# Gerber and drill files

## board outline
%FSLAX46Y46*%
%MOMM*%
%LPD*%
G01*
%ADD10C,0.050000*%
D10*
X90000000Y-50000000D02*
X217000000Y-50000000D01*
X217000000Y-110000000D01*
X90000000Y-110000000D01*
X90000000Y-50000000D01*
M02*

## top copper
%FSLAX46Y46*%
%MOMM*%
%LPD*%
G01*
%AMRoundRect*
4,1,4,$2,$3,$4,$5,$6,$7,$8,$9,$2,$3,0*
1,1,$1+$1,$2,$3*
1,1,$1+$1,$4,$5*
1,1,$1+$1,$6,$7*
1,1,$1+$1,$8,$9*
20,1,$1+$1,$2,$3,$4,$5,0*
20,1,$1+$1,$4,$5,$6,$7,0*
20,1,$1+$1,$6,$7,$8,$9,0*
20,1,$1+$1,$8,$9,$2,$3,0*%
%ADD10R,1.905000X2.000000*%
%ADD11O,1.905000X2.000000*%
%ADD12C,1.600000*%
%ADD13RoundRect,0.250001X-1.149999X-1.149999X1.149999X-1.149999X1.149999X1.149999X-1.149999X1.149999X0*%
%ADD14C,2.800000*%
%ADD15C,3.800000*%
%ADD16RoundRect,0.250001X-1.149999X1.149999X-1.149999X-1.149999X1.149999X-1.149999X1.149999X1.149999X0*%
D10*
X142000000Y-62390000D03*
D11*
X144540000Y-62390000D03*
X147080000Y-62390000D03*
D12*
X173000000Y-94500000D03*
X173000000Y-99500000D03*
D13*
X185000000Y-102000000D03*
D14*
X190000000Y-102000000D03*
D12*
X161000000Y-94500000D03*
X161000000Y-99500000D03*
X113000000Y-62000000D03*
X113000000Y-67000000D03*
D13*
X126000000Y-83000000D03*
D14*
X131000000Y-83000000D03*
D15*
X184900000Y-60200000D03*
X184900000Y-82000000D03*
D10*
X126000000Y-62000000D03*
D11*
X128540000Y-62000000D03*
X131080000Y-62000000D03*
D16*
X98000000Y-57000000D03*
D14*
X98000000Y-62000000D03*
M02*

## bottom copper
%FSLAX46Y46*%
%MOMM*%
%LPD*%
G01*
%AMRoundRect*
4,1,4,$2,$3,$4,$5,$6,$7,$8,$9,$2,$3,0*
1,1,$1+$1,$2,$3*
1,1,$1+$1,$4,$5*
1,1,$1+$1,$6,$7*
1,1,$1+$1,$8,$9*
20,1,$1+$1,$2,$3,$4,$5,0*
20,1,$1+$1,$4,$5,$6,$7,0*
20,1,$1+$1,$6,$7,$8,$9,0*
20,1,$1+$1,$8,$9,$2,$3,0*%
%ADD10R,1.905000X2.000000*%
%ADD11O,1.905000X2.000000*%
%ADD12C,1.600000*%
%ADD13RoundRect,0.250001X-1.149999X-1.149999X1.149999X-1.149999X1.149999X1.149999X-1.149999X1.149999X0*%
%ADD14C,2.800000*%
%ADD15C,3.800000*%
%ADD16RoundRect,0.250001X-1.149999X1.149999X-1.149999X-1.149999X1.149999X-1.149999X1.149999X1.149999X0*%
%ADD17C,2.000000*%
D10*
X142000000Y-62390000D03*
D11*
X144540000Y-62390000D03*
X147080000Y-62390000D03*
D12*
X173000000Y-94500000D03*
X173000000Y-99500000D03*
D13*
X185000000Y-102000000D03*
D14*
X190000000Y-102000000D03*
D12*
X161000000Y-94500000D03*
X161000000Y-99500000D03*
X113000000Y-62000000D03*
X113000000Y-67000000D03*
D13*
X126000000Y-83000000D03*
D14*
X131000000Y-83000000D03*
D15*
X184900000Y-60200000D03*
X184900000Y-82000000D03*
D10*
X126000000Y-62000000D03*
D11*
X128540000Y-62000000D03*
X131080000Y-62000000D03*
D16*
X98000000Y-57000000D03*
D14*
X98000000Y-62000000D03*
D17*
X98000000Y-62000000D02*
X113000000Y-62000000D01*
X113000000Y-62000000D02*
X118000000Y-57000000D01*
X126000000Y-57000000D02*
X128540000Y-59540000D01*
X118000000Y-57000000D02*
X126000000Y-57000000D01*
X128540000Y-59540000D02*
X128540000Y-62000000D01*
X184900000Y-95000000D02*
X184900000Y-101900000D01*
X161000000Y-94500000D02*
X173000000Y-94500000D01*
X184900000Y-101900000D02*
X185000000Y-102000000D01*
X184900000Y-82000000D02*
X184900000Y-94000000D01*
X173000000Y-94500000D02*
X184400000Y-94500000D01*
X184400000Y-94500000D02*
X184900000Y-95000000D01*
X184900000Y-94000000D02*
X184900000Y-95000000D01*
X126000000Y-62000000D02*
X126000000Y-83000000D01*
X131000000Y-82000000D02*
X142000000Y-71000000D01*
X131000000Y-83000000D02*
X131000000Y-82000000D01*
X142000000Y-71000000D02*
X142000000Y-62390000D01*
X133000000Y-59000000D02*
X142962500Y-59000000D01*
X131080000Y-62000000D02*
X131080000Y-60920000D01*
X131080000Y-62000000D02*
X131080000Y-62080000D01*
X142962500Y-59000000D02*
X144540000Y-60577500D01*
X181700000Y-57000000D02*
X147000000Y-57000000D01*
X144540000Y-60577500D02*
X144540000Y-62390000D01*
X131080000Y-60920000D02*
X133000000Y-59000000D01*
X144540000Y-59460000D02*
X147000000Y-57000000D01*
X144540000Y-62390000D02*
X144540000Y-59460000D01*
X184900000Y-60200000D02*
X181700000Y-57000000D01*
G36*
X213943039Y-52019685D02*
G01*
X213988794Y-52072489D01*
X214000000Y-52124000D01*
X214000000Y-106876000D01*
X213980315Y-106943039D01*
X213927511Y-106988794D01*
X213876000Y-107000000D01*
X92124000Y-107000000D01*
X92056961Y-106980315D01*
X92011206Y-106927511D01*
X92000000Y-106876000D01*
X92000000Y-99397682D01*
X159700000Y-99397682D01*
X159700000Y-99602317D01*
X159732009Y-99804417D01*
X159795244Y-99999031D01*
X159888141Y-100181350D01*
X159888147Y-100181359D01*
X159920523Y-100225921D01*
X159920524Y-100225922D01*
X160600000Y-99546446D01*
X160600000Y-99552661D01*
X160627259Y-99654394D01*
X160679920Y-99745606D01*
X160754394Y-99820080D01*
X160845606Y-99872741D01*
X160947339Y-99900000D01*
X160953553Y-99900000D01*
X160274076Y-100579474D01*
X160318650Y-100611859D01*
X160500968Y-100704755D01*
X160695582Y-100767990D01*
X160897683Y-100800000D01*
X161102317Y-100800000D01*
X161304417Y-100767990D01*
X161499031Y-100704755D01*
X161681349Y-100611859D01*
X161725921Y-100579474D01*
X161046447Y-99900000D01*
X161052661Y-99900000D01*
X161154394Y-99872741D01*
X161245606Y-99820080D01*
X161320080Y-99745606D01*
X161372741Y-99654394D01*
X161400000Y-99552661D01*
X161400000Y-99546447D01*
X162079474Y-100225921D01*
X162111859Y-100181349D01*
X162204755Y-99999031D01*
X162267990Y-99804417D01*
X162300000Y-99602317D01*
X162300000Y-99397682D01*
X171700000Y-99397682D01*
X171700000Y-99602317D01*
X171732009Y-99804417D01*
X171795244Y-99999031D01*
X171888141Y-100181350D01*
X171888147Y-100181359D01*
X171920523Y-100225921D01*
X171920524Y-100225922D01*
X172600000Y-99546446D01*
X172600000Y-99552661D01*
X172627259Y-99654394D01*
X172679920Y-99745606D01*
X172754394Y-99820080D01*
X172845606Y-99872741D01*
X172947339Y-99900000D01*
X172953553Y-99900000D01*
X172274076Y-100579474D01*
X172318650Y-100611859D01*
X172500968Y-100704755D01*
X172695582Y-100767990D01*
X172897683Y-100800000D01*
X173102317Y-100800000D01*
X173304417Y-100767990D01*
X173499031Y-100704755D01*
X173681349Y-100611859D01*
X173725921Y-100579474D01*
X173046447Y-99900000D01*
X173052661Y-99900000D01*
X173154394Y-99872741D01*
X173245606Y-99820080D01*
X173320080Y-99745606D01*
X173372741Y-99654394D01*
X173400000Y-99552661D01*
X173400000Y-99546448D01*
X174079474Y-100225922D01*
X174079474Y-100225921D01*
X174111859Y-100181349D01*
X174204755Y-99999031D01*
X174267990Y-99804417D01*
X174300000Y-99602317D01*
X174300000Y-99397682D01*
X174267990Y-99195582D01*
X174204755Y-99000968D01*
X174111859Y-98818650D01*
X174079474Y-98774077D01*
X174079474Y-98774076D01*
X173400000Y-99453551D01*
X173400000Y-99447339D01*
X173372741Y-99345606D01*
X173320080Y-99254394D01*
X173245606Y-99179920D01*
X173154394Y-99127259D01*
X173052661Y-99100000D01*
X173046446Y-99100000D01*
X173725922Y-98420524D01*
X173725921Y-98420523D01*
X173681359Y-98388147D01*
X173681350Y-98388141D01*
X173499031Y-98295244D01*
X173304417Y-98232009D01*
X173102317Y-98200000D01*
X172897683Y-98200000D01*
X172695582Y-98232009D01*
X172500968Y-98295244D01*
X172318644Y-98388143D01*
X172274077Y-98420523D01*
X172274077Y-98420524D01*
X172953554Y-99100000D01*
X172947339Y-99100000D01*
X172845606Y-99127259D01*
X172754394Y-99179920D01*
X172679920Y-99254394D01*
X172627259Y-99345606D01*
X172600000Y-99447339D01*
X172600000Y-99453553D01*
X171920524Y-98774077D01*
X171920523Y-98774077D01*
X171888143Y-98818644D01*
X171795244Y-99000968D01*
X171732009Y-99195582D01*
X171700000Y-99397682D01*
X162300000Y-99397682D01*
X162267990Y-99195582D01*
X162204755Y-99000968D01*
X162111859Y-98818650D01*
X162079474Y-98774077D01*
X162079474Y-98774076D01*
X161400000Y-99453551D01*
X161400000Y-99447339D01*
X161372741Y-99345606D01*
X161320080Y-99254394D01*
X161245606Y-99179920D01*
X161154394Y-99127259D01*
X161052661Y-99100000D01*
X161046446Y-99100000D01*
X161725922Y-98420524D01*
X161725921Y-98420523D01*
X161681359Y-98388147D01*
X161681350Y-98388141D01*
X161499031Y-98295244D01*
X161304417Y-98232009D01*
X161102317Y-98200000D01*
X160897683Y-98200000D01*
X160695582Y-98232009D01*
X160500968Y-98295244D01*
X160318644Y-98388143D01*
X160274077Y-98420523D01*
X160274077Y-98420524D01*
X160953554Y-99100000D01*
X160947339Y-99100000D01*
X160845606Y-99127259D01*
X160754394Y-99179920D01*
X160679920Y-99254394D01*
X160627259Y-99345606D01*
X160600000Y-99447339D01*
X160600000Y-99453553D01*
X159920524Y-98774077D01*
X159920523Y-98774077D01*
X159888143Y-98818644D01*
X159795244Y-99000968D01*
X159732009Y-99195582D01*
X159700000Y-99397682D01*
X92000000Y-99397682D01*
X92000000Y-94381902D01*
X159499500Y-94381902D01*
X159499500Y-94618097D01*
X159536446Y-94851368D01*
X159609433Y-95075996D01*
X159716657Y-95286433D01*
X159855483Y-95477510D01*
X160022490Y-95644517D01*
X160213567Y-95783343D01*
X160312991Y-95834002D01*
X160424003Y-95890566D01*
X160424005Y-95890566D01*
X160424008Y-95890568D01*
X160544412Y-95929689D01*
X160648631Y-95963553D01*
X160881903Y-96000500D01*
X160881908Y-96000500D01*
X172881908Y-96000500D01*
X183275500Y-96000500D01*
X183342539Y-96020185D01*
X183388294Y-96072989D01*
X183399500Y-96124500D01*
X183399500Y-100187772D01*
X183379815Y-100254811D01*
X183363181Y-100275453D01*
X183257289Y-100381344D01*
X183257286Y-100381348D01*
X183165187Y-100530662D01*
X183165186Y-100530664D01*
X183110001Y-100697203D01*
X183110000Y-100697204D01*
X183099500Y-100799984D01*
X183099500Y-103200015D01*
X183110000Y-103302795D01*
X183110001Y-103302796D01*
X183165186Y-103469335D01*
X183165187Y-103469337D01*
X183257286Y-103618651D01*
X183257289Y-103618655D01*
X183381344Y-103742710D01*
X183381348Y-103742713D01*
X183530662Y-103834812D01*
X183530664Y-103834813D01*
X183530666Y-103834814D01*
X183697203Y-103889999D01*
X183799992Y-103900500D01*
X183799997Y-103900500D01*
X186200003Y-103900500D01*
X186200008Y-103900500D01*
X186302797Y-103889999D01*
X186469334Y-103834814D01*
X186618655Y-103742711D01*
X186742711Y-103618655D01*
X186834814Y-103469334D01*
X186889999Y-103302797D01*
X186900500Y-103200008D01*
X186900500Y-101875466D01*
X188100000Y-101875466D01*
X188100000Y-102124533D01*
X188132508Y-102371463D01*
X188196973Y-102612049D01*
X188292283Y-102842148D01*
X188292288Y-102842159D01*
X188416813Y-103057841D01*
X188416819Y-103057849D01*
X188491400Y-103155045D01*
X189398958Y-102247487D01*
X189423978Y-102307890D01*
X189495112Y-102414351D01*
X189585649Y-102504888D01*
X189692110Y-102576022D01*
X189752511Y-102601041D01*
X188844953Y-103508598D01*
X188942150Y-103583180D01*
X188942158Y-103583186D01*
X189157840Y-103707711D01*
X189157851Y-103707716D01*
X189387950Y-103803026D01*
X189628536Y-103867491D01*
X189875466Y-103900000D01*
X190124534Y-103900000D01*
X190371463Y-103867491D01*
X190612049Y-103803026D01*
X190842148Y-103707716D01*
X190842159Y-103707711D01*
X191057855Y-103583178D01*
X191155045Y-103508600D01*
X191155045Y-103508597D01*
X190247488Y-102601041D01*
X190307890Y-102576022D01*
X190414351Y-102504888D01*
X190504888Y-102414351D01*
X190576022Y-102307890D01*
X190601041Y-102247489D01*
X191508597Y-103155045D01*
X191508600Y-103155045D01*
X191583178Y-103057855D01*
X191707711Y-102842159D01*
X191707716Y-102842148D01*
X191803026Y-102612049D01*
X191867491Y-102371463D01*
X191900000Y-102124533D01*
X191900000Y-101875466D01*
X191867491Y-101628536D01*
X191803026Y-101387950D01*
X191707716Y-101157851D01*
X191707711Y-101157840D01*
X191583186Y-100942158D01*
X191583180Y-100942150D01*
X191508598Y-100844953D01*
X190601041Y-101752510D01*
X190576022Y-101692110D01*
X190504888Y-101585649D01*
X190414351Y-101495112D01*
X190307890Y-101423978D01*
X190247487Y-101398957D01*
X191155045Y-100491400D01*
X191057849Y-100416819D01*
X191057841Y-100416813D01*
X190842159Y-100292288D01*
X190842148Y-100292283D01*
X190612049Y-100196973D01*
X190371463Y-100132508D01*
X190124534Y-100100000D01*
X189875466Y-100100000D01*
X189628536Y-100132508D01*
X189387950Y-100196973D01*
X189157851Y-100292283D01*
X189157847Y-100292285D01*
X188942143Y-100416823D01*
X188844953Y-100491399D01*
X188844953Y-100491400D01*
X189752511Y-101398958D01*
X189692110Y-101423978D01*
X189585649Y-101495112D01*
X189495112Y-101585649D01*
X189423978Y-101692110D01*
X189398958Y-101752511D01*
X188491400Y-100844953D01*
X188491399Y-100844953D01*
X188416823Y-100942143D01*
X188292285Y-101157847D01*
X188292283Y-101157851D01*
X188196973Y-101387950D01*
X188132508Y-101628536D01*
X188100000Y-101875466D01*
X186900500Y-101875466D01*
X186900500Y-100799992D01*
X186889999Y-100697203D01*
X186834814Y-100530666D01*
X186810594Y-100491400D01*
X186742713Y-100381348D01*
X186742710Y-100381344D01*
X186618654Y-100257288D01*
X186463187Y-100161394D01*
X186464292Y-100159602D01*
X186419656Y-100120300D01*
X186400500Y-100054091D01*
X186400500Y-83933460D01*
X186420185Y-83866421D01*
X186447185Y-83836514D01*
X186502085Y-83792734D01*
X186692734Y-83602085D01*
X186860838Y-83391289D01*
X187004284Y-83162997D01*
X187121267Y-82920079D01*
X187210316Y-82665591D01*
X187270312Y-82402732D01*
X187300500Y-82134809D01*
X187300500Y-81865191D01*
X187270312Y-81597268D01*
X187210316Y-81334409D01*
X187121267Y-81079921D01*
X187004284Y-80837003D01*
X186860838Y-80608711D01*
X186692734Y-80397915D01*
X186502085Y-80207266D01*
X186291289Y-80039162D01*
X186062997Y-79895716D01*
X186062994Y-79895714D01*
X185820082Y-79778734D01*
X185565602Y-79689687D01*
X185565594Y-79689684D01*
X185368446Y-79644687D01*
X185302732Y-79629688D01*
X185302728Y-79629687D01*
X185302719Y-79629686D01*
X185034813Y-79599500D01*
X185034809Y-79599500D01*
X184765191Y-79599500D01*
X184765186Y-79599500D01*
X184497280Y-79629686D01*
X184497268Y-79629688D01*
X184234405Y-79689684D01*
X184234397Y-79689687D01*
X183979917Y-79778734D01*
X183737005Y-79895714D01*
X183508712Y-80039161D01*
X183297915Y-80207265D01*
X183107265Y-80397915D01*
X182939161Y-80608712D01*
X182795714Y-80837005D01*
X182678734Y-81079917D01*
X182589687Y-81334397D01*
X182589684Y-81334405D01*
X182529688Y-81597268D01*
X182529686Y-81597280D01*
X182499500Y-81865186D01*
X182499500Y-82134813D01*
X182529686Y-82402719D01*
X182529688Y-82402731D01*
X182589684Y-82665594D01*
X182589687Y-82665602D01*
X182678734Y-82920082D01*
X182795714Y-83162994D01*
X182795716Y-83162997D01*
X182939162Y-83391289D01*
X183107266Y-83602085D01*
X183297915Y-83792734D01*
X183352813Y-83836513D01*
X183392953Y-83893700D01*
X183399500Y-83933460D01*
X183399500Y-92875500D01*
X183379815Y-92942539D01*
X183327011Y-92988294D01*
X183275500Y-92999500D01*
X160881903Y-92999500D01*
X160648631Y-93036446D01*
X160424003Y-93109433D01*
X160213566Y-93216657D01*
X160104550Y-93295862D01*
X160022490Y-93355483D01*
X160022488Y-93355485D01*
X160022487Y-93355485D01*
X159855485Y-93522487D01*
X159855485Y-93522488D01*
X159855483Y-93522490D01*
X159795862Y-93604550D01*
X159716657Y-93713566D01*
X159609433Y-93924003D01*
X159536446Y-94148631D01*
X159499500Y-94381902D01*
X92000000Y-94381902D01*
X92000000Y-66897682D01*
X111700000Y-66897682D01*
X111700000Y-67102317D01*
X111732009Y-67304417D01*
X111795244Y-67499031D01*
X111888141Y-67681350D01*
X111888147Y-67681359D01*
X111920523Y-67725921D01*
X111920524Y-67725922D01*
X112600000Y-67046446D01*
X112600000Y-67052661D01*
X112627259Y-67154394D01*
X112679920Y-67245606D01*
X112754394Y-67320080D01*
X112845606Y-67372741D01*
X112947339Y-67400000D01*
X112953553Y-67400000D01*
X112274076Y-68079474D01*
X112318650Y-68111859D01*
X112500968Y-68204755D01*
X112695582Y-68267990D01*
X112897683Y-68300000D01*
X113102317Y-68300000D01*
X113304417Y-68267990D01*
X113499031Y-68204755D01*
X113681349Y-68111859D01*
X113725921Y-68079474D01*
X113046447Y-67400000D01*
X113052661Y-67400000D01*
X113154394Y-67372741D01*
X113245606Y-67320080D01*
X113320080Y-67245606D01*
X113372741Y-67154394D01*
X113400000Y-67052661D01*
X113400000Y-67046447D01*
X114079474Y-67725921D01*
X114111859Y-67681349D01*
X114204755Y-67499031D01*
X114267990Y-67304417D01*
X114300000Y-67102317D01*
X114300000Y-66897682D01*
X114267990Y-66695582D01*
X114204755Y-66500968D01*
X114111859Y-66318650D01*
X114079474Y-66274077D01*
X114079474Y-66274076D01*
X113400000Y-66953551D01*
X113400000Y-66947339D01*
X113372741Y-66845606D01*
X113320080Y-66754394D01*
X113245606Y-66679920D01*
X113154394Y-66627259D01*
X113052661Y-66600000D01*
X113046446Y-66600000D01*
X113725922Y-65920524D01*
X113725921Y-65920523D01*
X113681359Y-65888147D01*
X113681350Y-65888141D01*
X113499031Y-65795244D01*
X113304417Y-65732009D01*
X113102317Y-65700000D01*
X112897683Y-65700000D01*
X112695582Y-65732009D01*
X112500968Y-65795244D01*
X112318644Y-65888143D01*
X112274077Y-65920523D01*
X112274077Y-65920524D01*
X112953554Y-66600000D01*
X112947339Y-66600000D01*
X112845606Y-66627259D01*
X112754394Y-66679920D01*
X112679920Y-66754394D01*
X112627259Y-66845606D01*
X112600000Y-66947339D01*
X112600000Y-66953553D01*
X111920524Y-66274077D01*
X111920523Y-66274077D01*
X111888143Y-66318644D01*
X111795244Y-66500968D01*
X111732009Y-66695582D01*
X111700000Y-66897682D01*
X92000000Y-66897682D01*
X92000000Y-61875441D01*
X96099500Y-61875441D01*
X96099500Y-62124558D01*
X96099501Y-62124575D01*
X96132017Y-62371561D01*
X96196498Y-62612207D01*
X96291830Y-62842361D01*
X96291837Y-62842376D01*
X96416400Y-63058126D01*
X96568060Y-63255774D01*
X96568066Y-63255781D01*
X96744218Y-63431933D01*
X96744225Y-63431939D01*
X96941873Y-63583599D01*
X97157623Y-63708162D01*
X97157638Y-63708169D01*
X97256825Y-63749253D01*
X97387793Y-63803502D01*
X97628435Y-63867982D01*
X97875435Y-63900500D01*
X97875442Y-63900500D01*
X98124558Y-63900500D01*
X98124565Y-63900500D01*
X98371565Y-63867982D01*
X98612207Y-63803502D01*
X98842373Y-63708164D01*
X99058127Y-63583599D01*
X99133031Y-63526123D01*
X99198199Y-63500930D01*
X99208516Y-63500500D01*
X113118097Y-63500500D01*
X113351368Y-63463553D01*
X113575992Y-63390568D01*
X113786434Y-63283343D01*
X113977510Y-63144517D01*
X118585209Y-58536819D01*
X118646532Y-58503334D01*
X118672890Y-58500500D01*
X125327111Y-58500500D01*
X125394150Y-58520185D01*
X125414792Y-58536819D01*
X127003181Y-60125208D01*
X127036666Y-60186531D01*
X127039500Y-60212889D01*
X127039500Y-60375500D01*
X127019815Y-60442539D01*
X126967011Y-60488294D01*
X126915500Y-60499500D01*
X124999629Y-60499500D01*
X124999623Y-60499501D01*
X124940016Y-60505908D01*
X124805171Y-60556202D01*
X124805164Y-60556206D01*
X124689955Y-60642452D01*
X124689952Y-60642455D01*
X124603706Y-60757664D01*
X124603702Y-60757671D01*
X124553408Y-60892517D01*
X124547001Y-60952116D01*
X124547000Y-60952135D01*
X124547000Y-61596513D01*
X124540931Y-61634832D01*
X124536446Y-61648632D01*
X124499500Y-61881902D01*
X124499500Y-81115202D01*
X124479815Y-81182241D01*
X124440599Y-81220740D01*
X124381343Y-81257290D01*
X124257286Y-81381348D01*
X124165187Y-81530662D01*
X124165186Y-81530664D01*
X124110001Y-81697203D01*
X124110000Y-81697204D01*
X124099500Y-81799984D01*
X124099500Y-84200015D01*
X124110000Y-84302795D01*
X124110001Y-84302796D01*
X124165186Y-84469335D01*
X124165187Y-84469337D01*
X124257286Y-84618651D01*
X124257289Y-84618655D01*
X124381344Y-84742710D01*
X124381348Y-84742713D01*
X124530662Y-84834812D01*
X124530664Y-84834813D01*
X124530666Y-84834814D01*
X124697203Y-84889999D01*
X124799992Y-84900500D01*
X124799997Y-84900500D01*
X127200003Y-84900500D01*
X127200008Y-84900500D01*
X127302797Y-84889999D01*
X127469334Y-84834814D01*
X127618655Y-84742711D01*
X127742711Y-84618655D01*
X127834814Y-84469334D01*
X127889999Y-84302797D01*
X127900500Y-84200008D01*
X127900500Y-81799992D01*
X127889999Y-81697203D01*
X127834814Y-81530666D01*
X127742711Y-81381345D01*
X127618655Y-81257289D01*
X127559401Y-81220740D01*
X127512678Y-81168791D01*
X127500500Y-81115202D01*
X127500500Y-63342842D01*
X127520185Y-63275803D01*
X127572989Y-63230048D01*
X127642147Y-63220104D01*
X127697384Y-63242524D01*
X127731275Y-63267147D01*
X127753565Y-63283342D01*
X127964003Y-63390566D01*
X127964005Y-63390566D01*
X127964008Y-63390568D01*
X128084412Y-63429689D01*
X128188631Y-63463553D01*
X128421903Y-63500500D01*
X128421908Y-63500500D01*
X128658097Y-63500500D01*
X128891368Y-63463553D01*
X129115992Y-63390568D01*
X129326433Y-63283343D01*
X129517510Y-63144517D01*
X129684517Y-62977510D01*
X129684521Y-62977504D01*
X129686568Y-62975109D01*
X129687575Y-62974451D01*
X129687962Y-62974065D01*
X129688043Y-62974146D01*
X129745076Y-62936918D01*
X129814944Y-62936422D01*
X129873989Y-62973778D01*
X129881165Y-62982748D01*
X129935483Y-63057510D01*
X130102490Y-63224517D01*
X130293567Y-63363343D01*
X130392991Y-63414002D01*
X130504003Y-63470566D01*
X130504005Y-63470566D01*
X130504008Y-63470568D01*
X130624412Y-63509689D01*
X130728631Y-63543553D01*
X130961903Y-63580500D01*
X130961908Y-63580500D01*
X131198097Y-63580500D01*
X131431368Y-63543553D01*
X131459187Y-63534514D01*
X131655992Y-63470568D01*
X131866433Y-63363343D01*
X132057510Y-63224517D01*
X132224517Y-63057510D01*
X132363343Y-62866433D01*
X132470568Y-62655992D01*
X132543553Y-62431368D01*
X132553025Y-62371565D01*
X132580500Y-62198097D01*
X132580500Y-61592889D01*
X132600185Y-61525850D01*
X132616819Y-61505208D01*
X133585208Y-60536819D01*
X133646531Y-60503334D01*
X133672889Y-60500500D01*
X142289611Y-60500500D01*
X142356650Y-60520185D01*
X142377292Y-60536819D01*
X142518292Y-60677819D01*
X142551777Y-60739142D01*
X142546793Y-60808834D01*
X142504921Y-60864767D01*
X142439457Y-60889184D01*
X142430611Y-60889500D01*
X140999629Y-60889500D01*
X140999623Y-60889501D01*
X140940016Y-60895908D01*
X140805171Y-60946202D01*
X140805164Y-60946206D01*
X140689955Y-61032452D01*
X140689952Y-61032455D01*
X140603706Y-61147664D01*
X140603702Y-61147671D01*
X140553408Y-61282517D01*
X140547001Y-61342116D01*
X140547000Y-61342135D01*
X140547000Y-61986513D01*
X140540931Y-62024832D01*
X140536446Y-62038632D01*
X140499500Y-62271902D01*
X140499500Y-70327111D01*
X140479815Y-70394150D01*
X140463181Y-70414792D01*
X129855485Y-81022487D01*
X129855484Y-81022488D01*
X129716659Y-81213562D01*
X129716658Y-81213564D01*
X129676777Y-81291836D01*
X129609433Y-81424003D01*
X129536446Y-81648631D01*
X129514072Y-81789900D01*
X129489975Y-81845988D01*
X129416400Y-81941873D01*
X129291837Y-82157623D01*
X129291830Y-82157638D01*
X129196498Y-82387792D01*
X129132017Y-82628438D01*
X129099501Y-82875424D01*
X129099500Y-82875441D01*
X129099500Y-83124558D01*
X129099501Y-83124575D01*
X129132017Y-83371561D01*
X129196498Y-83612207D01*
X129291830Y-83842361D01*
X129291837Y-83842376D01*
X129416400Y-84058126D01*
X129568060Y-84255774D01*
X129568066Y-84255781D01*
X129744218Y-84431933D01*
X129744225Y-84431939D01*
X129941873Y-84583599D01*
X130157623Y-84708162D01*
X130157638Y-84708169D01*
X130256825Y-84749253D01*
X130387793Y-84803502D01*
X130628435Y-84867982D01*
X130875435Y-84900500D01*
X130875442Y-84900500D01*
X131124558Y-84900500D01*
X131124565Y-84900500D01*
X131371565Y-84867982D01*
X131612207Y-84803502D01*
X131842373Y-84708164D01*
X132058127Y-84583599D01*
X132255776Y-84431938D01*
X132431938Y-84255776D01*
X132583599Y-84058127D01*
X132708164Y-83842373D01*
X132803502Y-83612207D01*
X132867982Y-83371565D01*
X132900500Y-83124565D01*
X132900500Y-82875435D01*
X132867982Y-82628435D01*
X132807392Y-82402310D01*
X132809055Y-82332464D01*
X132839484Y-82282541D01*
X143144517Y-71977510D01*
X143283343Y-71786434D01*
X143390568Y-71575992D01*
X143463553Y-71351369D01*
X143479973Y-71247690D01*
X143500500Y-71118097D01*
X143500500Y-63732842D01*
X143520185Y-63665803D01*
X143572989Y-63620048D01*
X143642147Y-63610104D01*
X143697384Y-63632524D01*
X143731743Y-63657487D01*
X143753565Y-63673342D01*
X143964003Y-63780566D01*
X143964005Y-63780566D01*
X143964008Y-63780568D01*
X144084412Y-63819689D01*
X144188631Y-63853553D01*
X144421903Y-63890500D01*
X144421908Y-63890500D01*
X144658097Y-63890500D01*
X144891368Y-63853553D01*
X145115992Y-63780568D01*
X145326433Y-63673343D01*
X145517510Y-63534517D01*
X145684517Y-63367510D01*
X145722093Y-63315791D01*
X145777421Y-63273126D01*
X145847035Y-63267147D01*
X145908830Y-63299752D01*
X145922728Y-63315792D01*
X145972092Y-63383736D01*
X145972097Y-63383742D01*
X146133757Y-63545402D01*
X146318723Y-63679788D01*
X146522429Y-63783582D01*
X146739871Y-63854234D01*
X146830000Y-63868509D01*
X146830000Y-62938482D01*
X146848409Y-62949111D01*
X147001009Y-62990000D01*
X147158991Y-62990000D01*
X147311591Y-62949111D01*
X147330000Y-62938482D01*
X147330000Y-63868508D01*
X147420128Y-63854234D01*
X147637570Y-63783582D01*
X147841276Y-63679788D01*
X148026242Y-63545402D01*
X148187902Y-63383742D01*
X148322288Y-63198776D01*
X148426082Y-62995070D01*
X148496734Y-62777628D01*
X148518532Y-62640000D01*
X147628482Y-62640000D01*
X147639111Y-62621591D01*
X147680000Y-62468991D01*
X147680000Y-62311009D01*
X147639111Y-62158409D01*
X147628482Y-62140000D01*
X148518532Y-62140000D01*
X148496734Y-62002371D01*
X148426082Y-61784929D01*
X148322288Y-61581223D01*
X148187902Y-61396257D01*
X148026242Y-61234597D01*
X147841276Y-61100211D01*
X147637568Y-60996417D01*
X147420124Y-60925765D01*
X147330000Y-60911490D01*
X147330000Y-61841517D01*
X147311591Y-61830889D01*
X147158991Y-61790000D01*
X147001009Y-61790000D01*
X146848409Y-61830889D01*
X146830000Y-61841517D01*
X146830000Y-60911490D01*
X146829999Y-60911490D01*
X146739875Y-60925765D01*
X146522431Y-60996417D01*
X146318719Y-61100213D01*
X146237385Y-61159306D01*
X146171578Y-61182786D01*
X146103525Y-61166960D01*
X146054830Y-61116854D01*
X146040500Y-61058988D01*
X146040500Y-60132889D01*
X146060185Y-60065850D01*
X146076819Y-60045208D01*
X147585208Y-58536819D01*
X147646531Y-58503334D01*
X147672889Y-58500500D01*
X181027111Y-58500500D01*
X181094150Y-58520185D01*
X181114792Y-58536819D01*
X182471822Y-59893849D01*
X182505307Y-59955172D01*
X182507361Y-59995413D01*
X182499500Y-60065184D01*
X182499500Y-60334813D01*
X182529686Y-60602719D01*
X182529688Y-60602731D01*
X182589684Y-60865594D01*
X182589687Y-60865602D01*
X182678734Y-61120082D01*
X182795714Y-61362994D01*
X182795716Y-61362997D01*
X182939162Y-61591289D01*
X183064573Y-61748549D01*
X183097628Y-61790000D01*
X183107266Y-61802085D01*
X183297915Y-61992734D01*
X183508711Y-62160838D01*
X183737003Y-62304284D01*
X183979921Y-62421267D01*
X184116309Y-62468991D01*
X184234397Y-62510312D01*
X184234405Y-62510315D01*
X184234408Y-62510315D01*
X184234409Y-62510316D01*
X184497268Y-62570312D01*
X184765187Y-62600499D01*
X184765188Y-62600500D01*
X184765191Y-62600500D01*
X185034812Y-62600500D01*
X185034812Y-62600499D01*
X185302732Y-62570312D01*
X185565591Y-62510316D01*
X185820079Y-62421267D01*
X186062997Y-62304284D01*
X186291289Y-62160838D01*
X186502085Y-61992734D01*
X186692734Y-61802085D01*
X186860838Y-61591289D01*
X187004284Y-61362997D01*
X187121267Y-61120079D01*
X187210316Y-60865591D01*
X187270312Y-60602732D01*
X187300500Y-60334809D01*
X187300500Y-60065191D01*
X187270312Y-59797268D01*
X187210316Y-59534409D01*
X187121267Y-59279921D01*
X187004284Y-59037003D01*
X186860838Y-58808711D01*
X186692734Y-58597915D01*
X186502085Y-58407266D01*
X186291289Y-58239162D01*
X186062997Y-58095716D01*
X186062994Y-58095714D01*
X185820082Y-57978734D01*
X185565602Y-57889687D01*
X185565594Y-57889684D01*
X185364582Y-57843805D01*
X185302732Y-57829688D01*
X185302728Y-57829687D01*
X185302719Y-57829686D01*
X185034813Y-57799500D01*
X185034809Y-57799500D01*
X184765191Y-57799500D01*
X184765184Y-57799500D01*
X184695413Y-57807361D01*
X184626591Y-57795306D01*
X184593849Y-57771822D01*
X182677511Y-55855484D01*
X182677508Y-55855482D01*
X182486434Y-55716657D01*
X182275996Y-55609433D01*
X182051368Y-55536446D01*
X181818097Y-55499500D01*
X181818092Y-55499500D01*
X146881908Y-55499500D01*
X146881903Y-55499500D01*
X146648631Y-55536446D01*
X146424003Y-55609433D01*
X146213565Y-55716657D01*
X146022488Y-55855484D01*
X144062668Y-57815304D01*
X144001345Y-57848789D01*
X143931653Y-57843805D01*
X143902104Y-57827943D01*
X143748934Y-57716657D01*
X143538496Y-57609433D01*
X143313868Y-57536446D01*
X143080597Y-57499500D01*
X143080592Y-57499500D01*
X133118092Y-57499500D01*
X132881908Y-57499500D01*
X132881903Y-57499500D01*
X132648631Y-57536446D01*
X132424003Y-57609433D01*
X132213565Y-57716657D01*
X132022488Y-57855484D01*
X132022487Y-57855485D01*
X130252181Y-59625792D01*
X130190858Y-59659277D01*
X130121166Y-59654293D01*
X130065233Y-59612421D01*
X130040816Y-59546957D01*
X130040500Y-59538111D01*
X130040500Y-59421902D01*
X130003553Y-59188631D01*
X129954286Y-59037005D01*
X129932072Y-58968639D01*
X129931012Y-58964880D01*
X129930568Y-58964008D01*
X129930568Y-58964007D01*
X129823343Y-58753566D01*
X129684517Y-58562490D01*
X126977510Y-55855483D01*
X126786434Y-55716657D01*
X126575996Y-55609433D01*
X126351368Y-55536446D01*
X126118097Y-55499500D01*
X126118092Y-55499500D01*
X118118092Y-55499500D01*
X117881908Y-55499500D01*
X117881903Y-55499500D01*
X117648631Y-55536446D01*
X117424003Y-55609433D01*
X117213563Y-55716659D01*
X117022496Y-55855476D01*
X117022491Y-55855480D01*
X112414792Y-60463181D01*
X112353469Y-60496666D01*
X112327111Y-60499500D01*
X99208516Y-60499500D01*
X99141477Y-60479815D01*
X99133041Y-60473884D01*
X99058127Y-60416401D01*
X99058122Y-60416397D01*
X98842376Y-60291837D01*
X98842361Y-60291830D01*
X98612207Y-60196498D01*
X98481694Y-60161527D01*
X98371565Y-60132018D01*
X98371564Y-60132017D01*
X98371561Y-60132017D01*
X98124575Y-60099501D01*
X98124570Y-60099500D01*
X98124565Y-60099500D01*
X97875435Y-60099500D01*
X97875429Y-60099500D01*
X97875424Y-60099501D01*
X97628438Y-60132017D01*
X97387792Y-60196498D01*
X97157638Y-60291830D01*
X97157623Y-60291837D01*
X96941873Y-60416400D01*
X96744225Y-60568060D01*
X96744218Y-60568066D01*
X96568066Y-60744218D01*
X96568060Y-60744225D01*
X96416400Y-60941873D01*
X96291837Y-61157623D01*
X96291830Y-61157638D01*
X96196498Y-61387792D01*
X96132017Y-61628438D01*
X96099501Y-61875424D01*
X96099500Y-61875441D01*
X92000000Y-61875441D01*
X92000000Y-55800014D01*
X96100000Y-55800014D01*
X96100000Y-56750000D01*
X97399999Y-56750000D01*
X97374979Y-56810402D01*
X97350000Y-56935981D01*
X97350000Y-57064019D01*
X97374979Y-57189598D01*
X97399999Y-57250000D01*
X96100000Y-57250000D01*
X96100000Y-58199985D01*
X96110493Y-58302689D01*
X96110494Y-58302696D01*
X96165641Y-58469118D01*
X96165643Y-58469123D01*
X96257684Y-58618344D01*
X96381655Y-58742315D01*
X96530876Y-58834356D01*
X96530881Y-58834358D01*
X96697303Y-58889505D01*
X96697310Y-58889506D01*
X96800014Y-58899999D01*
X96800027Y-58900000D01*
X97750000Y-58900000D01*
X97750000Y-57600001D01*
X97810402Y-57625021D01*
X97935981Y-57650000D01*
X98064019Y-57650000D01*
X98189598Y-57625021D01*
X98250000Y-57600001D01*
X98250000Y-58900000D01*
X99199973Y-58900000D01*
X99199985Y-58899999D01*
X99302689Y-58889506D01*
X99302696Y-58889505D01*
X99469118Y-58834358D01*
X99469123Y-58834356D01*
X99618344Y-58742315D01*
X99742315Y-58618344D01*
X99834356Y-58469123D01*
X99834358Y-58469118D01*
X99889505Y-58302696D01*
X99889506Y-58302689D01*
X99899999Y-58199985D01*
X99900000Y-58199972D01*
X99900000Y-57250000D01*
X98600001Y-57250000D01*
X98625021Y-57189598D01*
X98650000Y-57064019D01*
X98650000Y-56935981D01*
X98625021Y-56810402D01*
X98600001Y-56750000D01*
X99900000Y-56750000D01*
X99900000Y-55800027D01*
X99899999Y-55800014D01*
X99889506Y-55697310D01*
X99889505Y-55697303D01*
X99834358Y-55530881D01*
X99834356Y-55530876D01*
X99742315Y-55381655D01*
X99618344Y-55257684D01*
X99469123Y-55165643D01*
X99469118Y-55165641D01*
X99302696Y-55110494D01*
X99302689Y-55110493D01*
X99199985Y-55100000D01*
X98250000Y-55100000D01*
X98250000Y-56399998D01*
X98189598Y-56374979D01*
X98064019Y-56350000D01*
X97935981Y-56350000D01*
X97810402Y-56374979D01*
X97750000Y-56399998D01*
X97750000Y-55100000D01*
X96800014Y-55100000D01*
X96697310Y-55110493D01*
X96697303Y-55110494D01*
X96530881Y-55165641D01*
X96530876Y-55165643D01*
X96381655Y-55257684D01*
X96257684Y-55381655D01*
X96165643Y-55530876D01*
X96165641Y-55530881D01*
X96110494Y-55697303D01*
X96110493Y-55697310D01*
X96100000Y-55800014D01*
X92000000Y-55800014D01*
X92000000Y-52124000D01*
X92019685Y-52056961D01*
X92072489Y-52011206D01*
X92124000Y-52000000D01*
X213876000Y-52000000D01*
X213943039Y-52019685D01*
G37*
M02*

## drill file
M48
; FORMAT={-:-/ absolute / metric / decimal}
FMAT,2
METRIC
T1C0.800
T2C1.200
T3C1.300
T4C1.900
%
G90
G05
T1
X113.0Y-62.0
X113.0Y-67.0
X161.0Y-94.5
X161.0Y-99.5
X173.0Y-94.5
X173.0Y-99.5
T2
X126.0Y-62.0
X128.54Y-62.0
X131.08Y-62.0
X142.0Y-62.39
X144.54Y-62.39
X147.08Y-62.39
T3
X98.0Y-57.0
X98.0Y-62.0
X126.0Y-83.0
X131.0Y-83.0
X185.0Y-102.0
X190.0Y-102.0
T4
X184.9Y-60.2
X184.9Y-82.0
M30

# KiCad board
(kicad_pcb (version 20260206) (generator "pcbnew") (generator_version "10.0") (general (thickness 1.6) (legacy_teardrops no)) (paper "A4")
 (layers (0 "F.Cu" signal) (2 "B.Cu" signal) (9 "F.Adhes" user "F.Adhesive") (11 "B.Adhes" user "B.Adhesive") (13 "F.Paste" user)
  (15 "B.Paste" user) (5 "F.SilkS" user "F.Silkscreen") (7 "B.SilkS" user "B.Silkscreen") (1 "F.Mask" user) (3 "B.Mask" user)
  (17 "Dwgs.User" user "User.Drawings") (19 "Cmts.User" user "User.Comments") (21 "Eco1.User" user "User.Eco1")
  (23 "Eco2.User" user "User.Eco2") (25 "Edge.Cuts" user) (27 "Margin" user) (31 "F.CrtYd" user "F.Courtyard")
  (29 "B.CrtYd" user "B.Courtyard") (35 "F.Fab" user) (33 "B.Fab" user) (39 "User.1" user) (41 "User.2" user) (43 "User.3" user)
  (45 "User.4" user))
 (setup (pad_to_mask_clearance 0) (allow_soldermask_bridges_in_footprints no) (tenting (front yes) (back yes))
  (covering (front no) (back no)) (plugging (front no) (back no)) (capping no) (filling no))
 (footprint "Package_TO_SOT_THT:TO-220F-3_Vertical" (layer "F.Cu") (at 142 62.39)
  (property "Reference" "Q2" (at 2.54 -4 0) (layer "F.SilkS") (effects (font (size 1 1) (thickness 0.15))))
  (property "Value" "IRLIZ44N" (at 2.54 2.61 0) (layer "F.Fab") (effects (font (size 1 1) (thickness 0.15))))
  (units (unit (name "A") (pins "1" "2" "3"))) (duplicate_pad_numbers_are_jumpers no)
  (pad "1" thru_hole rect (at 0 0) (size 1.905 2) (drill 1.2) (layers "*.Cu" "*.Mask") (remove_unused_layers no) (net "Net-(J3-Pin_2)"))
  (pad "2" thru_hole oval (at 2.54 0) (size 1.905 2) (drill 1.2) (layers "*.Cu" "*.Mask") (remove_unused_layers no) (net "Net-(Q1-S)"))
  (pad "3" thru_hole oval (at 5.08 0) (size 1.905 2) (drill 1.2) (layers "*.Cu" "*.Mask") (remove_unused_layers no) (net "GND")))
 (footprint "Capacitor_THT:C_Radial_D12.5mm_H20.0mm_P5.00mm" (layer "F.Cu") (at 173 94.5 -90)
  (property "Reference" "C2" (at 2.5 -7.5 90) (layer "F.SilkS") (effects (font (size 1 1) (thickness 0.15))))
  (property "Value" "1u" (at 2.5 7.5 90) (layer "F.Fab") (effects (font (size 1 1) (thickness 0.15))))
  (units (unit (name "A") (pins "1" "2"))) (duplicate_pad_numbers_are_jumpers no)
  (pad "1" thru_hole circle (at 0 0 270) (size 1.6 1.6) (drill 0.8) (layers "*.Cu" "*.Mask") (remove_unused_layers no)
   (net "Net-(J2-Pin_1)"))
  (pad "2" thru_hole circle (at 5 0 270) (size 1.6 1.6) (drill 0.8) (layers "*.Cu" "*.Mask") (remove_unused_layers no) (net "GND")))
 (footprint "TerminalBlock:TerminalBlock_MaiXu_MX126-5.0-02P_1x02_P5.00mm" (layer "F.Cu") (at 185 102)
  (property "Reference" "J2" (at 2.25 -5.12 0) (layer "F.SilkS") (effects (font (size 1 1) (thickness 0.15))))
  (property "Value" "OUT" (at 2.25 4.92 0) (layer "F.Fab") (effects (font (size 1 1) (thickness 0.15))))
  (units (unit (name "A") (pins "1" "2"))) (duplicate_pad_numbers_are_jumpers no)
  (pad "1" thru_hole roundrect (at 0 0) (size 2.8 2.8) (drill 1.3) (layers "*.Cu" "*.Mask") (remove_unused_layers no)
   (roundrect_rratio 0.089286) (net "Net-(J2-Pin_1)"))
  (pad "2" thru_hole circle (at 5 0) (size 2.8 2.8) (drill 1.3) (layers "*.Cu" "*.Mask") (remove_unused_layers no) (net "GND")))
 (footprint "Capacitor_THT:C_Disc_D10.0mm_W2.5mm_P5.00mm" (layer "F.Cu") (at 161 94.5 -90)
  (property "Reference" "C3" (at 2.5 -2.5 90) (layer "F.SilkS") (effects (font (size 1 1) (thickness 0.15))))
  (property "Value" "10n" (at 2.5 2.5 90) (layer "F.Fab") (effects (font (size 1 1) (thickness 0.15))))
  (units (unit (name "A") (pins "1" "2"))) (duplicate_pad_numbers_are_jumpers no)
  (pad "1" thru_hole circle (at 0 0 270) (size 1.6 1.6) (drill 0.8) (layers "*.Cu" "*.Mask") (remove_unused_layers no)
   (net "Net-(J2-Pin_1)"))
  (pad "2" thru_hole circle (at 5 0 270) (size 1.6 1.6) (drill 0.8) (layers "*.Cu" "*.Mask") (remove_unused_layers no) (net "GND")))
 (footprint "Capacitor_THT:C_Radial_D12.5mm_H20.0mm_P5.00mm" (layer "F.Cu") (at 113 62 -90)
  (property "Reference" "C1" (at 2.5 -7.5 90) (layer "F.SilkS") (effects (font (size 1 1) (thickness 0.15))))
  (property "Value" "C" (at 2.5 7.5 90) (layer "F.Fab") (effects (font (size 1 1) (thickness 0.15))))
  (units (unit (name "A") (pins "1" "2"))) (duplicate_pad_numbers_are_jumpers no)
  (pad "1" thru_hole circle (at 0 0 270) (size 1.6 1.6) (drill 0.8) (layers "*.Cu" "*.Mask") (remove_unused_layers no)
   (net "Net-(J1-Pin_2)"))
  (pad "2" thru_hole circle (at 5 0 270) (size 1.6 1.6) (drill 0.8) (layers "*.Cu" "*.Mask") (remove_unused_layers no) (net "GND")))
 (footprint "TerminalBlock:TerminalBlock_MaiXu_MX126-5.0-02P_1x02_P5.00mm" (layer "F.Cu") (at 126 83)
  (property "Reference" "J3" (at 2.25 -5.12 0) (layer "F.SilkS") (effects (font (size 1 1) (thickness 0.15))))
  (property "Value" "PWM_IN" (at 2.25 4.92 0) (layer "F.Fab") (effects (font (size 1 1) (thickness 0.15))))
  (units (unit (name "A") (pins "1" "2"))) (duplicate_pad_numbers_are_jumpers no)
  (pad "1" thru_hole roundrect (at 0 0) (size 2.8 2.8) (drill 1.3) (layers "*.Cu" "*.Mask") (remove_unused_layers no)
   (roundrect_rratio 0.089286) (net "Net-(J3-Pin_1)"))
  (pad "2" thru_hole circle (at 5 0) (size 2.8 2.8) (drill 1.3) (layers "*.Cu" "*.Mask") (remove_unused_layers no) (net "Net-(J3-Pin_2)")))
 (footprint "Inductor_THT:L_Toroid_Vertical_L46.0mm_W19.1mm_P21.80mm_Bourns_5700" (layer "F.Cu") (at 184.9 60.2)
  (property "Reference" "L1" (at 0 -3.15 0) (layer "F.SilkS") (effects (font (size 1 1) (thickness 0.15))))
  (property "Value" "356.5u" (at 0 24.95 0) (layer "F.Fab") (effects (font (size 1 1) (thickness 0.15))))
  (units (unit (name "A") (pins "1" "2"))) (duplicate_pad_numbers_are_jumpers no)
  (pad "1" thru_hole circle (at 0 0) (size 3.8 3.8) (drill 1.9) (layers "*.Cu" "*.Mask") (remove_unused_layers no) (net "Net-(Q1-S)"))
  (pad "2" thru_hole circle (at 0 21.8) (size 3.8 3.8) (drill 1.9) (layers "*.Cu" "*.Mask") (remove_unused_layers no) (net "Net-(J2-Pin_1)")))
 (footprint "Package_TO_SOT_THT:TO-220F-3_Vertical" (layer "F.Cu") (at 126 62)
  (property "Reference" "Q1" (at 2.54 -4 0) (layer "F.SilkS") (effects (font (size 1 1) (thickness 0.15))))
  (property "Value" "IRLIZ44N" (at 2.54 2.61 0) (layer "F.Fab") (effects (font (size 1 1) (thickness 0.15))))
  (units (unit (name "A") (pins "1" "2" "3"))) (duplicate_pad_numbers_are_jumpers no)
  (pad "1" thru_hole rect (at 0 0) (size 1.905 2) (drill 1.2) (layers "*.Cu" "*.Mask") (remove_unused_layers no) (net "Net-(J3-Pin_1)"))
  (pad "2" thru_hole oval (at 2.54 0) (size 1.905 2) (drill 1.2) (layers "*.Cu" "*.Mask") (remove_unused_layers no) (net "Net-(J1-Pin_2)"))
  (pad "3" thru_hole oval (at 5.08 0) (size 1.905 2) (drill 1.2) (layers "*.Cu" "*.Mask") (remove_unused_layers no) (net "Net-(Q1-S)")))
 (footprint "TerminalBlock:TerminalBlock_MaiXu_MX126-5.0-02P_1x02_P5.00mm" (layer "F.Cu") (at 98 57 -90)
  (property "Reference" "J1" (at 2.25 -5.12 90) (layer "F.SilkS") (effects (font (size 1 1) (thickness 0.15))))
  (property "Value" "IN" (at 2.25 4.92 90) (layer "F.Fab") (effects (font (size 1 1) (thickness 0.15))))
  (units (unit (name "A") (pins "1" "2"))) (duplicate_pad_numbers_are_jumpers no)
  (pad "1" thru_hole roundrect (at 0 0 270) (size 2.8 2.8) (drill 1.3) (layers "*.Cu" "*.Mask") (remove_unused_layers no)
   (roundrect_rratio 0.089286) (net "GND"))
  (pad "2" thru_hole circle (at 5 0 270) (size 2.8 2.8) (drill 1.3) (layers "*.Cu" "*.Mask") (remove_unused_layers no)
   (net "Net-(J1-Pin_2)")))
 (gr_rect (start 90 50) (end 217 110) (stroke (width 0.05) (type default)) (fill no) (layer "Edge.Cuts"))
 (segment (start 98 62) (end 113 62) (width 2) (layer "B.Cu") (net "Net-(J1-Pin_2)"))
 (segment (start 113 62) (end 118 57) (width 2) (layer "B.Cu") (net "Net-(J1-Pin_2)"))
 (segment (start 126 57) (end 128.54 59.54) (width 2) (layer "B.Cu") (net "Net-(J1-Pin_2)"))
 (segment (start 118 57) (end 126 57) (width 2) (layer "B.Cu") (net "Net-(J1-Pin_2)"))
 (segment (start 128.54 59.54) (end 128.54 62) (width 2) (layer "B.Cu") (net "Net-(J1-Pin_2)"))
 (segment (start 184.9 95) (end 184.9 101.9) (width 2) (layer "B.Cu") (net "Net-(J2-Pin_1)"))
 (segment (start 161 94.5) (end 173 94.5) (width 2) (layer "B.Cu") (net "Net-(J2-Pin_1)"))
 (segment (start 184.9 101.9) (end 185 102) (width 2) (layer "B.Cu") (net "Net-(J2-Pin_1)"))
 (segment (start 184.9 82) (end 184.9 94) (width 2) (layer "B.Cu") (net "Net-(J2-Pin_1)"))
 (segment (start 173 94.5) (end 184.4 94.5) (width 2) (layer "B.Cu") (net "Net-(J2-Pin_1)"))
 (segment (start 184.4 94.5) (end 184.9 95) (width 2) (layer "B.Cu") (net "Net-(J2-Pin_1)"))
 (segment (start 184.9 94) (end 184.9 95) (width 2) (layer "B.Cu") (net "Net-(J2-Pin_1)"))
 (segment (start 126 62) (end 126 83) (width 2) (layer "B.Cu") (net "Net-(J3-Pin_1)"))
 (segment (start 131 82) (end 142 71) (width 2) (layer "B.Cu") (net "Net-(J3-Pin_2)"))
 (segment (start 131 83) (end 131 82) (width 2) (layer "B.Cu") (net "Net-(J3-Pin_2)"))
 (segment (start 142 71) (end 142 62.39) (width 2) (layer "B.Cu") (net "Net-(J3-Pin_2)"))
 (segment (start 133 59) (end 142.9625 59) (width 2) (layer "B.Cu") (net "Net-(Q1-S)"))
 (segment (start 131.08 62) (end 131.08 60.92) (width 2) (layer "B.Cu") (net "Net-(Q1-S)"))
 (segment (start 131.08 62) (end 131.08 62.08) (width 2) (layer "B.Cu") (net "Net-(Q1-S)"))
 (segment (start 142.9625 59) (end 144.54 60.5775) (width 2) (layer "B.Cu") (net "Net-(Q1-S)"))
 (segment (start 181.7 57) (end 147 57) (width 2) (layer "B.Cu") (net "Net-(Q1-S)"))
 (segment (start 144.54 60.5775) (end 144.54 62.39) (width 2) (layer "B.Cu") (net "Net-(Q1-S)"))
 (segment (start 131.08 60.92) (end 133 59) (width 2) (layer "B.Cu") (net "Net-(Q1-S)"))
 (segment (start 144.54 59.46) (end 147 57) (width 2) (layer "B.Cu") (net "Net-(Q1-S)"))
 (segment (start 144.54 62.39) (end 144.54 59.46) (width 2) (layer "B.Cu") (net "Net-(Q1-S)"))
 (segment (start 184.9 60.2) (end 181.7 57) (width 2) (layer "B.Cu") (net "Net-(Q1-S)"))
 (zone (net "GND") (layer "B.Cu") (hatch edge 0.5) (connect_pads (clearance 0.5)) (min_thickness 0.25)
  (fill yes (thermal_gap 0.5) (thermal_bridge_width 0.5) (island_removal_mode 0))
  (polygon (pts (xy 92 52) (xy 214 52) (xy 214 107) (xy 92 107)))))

